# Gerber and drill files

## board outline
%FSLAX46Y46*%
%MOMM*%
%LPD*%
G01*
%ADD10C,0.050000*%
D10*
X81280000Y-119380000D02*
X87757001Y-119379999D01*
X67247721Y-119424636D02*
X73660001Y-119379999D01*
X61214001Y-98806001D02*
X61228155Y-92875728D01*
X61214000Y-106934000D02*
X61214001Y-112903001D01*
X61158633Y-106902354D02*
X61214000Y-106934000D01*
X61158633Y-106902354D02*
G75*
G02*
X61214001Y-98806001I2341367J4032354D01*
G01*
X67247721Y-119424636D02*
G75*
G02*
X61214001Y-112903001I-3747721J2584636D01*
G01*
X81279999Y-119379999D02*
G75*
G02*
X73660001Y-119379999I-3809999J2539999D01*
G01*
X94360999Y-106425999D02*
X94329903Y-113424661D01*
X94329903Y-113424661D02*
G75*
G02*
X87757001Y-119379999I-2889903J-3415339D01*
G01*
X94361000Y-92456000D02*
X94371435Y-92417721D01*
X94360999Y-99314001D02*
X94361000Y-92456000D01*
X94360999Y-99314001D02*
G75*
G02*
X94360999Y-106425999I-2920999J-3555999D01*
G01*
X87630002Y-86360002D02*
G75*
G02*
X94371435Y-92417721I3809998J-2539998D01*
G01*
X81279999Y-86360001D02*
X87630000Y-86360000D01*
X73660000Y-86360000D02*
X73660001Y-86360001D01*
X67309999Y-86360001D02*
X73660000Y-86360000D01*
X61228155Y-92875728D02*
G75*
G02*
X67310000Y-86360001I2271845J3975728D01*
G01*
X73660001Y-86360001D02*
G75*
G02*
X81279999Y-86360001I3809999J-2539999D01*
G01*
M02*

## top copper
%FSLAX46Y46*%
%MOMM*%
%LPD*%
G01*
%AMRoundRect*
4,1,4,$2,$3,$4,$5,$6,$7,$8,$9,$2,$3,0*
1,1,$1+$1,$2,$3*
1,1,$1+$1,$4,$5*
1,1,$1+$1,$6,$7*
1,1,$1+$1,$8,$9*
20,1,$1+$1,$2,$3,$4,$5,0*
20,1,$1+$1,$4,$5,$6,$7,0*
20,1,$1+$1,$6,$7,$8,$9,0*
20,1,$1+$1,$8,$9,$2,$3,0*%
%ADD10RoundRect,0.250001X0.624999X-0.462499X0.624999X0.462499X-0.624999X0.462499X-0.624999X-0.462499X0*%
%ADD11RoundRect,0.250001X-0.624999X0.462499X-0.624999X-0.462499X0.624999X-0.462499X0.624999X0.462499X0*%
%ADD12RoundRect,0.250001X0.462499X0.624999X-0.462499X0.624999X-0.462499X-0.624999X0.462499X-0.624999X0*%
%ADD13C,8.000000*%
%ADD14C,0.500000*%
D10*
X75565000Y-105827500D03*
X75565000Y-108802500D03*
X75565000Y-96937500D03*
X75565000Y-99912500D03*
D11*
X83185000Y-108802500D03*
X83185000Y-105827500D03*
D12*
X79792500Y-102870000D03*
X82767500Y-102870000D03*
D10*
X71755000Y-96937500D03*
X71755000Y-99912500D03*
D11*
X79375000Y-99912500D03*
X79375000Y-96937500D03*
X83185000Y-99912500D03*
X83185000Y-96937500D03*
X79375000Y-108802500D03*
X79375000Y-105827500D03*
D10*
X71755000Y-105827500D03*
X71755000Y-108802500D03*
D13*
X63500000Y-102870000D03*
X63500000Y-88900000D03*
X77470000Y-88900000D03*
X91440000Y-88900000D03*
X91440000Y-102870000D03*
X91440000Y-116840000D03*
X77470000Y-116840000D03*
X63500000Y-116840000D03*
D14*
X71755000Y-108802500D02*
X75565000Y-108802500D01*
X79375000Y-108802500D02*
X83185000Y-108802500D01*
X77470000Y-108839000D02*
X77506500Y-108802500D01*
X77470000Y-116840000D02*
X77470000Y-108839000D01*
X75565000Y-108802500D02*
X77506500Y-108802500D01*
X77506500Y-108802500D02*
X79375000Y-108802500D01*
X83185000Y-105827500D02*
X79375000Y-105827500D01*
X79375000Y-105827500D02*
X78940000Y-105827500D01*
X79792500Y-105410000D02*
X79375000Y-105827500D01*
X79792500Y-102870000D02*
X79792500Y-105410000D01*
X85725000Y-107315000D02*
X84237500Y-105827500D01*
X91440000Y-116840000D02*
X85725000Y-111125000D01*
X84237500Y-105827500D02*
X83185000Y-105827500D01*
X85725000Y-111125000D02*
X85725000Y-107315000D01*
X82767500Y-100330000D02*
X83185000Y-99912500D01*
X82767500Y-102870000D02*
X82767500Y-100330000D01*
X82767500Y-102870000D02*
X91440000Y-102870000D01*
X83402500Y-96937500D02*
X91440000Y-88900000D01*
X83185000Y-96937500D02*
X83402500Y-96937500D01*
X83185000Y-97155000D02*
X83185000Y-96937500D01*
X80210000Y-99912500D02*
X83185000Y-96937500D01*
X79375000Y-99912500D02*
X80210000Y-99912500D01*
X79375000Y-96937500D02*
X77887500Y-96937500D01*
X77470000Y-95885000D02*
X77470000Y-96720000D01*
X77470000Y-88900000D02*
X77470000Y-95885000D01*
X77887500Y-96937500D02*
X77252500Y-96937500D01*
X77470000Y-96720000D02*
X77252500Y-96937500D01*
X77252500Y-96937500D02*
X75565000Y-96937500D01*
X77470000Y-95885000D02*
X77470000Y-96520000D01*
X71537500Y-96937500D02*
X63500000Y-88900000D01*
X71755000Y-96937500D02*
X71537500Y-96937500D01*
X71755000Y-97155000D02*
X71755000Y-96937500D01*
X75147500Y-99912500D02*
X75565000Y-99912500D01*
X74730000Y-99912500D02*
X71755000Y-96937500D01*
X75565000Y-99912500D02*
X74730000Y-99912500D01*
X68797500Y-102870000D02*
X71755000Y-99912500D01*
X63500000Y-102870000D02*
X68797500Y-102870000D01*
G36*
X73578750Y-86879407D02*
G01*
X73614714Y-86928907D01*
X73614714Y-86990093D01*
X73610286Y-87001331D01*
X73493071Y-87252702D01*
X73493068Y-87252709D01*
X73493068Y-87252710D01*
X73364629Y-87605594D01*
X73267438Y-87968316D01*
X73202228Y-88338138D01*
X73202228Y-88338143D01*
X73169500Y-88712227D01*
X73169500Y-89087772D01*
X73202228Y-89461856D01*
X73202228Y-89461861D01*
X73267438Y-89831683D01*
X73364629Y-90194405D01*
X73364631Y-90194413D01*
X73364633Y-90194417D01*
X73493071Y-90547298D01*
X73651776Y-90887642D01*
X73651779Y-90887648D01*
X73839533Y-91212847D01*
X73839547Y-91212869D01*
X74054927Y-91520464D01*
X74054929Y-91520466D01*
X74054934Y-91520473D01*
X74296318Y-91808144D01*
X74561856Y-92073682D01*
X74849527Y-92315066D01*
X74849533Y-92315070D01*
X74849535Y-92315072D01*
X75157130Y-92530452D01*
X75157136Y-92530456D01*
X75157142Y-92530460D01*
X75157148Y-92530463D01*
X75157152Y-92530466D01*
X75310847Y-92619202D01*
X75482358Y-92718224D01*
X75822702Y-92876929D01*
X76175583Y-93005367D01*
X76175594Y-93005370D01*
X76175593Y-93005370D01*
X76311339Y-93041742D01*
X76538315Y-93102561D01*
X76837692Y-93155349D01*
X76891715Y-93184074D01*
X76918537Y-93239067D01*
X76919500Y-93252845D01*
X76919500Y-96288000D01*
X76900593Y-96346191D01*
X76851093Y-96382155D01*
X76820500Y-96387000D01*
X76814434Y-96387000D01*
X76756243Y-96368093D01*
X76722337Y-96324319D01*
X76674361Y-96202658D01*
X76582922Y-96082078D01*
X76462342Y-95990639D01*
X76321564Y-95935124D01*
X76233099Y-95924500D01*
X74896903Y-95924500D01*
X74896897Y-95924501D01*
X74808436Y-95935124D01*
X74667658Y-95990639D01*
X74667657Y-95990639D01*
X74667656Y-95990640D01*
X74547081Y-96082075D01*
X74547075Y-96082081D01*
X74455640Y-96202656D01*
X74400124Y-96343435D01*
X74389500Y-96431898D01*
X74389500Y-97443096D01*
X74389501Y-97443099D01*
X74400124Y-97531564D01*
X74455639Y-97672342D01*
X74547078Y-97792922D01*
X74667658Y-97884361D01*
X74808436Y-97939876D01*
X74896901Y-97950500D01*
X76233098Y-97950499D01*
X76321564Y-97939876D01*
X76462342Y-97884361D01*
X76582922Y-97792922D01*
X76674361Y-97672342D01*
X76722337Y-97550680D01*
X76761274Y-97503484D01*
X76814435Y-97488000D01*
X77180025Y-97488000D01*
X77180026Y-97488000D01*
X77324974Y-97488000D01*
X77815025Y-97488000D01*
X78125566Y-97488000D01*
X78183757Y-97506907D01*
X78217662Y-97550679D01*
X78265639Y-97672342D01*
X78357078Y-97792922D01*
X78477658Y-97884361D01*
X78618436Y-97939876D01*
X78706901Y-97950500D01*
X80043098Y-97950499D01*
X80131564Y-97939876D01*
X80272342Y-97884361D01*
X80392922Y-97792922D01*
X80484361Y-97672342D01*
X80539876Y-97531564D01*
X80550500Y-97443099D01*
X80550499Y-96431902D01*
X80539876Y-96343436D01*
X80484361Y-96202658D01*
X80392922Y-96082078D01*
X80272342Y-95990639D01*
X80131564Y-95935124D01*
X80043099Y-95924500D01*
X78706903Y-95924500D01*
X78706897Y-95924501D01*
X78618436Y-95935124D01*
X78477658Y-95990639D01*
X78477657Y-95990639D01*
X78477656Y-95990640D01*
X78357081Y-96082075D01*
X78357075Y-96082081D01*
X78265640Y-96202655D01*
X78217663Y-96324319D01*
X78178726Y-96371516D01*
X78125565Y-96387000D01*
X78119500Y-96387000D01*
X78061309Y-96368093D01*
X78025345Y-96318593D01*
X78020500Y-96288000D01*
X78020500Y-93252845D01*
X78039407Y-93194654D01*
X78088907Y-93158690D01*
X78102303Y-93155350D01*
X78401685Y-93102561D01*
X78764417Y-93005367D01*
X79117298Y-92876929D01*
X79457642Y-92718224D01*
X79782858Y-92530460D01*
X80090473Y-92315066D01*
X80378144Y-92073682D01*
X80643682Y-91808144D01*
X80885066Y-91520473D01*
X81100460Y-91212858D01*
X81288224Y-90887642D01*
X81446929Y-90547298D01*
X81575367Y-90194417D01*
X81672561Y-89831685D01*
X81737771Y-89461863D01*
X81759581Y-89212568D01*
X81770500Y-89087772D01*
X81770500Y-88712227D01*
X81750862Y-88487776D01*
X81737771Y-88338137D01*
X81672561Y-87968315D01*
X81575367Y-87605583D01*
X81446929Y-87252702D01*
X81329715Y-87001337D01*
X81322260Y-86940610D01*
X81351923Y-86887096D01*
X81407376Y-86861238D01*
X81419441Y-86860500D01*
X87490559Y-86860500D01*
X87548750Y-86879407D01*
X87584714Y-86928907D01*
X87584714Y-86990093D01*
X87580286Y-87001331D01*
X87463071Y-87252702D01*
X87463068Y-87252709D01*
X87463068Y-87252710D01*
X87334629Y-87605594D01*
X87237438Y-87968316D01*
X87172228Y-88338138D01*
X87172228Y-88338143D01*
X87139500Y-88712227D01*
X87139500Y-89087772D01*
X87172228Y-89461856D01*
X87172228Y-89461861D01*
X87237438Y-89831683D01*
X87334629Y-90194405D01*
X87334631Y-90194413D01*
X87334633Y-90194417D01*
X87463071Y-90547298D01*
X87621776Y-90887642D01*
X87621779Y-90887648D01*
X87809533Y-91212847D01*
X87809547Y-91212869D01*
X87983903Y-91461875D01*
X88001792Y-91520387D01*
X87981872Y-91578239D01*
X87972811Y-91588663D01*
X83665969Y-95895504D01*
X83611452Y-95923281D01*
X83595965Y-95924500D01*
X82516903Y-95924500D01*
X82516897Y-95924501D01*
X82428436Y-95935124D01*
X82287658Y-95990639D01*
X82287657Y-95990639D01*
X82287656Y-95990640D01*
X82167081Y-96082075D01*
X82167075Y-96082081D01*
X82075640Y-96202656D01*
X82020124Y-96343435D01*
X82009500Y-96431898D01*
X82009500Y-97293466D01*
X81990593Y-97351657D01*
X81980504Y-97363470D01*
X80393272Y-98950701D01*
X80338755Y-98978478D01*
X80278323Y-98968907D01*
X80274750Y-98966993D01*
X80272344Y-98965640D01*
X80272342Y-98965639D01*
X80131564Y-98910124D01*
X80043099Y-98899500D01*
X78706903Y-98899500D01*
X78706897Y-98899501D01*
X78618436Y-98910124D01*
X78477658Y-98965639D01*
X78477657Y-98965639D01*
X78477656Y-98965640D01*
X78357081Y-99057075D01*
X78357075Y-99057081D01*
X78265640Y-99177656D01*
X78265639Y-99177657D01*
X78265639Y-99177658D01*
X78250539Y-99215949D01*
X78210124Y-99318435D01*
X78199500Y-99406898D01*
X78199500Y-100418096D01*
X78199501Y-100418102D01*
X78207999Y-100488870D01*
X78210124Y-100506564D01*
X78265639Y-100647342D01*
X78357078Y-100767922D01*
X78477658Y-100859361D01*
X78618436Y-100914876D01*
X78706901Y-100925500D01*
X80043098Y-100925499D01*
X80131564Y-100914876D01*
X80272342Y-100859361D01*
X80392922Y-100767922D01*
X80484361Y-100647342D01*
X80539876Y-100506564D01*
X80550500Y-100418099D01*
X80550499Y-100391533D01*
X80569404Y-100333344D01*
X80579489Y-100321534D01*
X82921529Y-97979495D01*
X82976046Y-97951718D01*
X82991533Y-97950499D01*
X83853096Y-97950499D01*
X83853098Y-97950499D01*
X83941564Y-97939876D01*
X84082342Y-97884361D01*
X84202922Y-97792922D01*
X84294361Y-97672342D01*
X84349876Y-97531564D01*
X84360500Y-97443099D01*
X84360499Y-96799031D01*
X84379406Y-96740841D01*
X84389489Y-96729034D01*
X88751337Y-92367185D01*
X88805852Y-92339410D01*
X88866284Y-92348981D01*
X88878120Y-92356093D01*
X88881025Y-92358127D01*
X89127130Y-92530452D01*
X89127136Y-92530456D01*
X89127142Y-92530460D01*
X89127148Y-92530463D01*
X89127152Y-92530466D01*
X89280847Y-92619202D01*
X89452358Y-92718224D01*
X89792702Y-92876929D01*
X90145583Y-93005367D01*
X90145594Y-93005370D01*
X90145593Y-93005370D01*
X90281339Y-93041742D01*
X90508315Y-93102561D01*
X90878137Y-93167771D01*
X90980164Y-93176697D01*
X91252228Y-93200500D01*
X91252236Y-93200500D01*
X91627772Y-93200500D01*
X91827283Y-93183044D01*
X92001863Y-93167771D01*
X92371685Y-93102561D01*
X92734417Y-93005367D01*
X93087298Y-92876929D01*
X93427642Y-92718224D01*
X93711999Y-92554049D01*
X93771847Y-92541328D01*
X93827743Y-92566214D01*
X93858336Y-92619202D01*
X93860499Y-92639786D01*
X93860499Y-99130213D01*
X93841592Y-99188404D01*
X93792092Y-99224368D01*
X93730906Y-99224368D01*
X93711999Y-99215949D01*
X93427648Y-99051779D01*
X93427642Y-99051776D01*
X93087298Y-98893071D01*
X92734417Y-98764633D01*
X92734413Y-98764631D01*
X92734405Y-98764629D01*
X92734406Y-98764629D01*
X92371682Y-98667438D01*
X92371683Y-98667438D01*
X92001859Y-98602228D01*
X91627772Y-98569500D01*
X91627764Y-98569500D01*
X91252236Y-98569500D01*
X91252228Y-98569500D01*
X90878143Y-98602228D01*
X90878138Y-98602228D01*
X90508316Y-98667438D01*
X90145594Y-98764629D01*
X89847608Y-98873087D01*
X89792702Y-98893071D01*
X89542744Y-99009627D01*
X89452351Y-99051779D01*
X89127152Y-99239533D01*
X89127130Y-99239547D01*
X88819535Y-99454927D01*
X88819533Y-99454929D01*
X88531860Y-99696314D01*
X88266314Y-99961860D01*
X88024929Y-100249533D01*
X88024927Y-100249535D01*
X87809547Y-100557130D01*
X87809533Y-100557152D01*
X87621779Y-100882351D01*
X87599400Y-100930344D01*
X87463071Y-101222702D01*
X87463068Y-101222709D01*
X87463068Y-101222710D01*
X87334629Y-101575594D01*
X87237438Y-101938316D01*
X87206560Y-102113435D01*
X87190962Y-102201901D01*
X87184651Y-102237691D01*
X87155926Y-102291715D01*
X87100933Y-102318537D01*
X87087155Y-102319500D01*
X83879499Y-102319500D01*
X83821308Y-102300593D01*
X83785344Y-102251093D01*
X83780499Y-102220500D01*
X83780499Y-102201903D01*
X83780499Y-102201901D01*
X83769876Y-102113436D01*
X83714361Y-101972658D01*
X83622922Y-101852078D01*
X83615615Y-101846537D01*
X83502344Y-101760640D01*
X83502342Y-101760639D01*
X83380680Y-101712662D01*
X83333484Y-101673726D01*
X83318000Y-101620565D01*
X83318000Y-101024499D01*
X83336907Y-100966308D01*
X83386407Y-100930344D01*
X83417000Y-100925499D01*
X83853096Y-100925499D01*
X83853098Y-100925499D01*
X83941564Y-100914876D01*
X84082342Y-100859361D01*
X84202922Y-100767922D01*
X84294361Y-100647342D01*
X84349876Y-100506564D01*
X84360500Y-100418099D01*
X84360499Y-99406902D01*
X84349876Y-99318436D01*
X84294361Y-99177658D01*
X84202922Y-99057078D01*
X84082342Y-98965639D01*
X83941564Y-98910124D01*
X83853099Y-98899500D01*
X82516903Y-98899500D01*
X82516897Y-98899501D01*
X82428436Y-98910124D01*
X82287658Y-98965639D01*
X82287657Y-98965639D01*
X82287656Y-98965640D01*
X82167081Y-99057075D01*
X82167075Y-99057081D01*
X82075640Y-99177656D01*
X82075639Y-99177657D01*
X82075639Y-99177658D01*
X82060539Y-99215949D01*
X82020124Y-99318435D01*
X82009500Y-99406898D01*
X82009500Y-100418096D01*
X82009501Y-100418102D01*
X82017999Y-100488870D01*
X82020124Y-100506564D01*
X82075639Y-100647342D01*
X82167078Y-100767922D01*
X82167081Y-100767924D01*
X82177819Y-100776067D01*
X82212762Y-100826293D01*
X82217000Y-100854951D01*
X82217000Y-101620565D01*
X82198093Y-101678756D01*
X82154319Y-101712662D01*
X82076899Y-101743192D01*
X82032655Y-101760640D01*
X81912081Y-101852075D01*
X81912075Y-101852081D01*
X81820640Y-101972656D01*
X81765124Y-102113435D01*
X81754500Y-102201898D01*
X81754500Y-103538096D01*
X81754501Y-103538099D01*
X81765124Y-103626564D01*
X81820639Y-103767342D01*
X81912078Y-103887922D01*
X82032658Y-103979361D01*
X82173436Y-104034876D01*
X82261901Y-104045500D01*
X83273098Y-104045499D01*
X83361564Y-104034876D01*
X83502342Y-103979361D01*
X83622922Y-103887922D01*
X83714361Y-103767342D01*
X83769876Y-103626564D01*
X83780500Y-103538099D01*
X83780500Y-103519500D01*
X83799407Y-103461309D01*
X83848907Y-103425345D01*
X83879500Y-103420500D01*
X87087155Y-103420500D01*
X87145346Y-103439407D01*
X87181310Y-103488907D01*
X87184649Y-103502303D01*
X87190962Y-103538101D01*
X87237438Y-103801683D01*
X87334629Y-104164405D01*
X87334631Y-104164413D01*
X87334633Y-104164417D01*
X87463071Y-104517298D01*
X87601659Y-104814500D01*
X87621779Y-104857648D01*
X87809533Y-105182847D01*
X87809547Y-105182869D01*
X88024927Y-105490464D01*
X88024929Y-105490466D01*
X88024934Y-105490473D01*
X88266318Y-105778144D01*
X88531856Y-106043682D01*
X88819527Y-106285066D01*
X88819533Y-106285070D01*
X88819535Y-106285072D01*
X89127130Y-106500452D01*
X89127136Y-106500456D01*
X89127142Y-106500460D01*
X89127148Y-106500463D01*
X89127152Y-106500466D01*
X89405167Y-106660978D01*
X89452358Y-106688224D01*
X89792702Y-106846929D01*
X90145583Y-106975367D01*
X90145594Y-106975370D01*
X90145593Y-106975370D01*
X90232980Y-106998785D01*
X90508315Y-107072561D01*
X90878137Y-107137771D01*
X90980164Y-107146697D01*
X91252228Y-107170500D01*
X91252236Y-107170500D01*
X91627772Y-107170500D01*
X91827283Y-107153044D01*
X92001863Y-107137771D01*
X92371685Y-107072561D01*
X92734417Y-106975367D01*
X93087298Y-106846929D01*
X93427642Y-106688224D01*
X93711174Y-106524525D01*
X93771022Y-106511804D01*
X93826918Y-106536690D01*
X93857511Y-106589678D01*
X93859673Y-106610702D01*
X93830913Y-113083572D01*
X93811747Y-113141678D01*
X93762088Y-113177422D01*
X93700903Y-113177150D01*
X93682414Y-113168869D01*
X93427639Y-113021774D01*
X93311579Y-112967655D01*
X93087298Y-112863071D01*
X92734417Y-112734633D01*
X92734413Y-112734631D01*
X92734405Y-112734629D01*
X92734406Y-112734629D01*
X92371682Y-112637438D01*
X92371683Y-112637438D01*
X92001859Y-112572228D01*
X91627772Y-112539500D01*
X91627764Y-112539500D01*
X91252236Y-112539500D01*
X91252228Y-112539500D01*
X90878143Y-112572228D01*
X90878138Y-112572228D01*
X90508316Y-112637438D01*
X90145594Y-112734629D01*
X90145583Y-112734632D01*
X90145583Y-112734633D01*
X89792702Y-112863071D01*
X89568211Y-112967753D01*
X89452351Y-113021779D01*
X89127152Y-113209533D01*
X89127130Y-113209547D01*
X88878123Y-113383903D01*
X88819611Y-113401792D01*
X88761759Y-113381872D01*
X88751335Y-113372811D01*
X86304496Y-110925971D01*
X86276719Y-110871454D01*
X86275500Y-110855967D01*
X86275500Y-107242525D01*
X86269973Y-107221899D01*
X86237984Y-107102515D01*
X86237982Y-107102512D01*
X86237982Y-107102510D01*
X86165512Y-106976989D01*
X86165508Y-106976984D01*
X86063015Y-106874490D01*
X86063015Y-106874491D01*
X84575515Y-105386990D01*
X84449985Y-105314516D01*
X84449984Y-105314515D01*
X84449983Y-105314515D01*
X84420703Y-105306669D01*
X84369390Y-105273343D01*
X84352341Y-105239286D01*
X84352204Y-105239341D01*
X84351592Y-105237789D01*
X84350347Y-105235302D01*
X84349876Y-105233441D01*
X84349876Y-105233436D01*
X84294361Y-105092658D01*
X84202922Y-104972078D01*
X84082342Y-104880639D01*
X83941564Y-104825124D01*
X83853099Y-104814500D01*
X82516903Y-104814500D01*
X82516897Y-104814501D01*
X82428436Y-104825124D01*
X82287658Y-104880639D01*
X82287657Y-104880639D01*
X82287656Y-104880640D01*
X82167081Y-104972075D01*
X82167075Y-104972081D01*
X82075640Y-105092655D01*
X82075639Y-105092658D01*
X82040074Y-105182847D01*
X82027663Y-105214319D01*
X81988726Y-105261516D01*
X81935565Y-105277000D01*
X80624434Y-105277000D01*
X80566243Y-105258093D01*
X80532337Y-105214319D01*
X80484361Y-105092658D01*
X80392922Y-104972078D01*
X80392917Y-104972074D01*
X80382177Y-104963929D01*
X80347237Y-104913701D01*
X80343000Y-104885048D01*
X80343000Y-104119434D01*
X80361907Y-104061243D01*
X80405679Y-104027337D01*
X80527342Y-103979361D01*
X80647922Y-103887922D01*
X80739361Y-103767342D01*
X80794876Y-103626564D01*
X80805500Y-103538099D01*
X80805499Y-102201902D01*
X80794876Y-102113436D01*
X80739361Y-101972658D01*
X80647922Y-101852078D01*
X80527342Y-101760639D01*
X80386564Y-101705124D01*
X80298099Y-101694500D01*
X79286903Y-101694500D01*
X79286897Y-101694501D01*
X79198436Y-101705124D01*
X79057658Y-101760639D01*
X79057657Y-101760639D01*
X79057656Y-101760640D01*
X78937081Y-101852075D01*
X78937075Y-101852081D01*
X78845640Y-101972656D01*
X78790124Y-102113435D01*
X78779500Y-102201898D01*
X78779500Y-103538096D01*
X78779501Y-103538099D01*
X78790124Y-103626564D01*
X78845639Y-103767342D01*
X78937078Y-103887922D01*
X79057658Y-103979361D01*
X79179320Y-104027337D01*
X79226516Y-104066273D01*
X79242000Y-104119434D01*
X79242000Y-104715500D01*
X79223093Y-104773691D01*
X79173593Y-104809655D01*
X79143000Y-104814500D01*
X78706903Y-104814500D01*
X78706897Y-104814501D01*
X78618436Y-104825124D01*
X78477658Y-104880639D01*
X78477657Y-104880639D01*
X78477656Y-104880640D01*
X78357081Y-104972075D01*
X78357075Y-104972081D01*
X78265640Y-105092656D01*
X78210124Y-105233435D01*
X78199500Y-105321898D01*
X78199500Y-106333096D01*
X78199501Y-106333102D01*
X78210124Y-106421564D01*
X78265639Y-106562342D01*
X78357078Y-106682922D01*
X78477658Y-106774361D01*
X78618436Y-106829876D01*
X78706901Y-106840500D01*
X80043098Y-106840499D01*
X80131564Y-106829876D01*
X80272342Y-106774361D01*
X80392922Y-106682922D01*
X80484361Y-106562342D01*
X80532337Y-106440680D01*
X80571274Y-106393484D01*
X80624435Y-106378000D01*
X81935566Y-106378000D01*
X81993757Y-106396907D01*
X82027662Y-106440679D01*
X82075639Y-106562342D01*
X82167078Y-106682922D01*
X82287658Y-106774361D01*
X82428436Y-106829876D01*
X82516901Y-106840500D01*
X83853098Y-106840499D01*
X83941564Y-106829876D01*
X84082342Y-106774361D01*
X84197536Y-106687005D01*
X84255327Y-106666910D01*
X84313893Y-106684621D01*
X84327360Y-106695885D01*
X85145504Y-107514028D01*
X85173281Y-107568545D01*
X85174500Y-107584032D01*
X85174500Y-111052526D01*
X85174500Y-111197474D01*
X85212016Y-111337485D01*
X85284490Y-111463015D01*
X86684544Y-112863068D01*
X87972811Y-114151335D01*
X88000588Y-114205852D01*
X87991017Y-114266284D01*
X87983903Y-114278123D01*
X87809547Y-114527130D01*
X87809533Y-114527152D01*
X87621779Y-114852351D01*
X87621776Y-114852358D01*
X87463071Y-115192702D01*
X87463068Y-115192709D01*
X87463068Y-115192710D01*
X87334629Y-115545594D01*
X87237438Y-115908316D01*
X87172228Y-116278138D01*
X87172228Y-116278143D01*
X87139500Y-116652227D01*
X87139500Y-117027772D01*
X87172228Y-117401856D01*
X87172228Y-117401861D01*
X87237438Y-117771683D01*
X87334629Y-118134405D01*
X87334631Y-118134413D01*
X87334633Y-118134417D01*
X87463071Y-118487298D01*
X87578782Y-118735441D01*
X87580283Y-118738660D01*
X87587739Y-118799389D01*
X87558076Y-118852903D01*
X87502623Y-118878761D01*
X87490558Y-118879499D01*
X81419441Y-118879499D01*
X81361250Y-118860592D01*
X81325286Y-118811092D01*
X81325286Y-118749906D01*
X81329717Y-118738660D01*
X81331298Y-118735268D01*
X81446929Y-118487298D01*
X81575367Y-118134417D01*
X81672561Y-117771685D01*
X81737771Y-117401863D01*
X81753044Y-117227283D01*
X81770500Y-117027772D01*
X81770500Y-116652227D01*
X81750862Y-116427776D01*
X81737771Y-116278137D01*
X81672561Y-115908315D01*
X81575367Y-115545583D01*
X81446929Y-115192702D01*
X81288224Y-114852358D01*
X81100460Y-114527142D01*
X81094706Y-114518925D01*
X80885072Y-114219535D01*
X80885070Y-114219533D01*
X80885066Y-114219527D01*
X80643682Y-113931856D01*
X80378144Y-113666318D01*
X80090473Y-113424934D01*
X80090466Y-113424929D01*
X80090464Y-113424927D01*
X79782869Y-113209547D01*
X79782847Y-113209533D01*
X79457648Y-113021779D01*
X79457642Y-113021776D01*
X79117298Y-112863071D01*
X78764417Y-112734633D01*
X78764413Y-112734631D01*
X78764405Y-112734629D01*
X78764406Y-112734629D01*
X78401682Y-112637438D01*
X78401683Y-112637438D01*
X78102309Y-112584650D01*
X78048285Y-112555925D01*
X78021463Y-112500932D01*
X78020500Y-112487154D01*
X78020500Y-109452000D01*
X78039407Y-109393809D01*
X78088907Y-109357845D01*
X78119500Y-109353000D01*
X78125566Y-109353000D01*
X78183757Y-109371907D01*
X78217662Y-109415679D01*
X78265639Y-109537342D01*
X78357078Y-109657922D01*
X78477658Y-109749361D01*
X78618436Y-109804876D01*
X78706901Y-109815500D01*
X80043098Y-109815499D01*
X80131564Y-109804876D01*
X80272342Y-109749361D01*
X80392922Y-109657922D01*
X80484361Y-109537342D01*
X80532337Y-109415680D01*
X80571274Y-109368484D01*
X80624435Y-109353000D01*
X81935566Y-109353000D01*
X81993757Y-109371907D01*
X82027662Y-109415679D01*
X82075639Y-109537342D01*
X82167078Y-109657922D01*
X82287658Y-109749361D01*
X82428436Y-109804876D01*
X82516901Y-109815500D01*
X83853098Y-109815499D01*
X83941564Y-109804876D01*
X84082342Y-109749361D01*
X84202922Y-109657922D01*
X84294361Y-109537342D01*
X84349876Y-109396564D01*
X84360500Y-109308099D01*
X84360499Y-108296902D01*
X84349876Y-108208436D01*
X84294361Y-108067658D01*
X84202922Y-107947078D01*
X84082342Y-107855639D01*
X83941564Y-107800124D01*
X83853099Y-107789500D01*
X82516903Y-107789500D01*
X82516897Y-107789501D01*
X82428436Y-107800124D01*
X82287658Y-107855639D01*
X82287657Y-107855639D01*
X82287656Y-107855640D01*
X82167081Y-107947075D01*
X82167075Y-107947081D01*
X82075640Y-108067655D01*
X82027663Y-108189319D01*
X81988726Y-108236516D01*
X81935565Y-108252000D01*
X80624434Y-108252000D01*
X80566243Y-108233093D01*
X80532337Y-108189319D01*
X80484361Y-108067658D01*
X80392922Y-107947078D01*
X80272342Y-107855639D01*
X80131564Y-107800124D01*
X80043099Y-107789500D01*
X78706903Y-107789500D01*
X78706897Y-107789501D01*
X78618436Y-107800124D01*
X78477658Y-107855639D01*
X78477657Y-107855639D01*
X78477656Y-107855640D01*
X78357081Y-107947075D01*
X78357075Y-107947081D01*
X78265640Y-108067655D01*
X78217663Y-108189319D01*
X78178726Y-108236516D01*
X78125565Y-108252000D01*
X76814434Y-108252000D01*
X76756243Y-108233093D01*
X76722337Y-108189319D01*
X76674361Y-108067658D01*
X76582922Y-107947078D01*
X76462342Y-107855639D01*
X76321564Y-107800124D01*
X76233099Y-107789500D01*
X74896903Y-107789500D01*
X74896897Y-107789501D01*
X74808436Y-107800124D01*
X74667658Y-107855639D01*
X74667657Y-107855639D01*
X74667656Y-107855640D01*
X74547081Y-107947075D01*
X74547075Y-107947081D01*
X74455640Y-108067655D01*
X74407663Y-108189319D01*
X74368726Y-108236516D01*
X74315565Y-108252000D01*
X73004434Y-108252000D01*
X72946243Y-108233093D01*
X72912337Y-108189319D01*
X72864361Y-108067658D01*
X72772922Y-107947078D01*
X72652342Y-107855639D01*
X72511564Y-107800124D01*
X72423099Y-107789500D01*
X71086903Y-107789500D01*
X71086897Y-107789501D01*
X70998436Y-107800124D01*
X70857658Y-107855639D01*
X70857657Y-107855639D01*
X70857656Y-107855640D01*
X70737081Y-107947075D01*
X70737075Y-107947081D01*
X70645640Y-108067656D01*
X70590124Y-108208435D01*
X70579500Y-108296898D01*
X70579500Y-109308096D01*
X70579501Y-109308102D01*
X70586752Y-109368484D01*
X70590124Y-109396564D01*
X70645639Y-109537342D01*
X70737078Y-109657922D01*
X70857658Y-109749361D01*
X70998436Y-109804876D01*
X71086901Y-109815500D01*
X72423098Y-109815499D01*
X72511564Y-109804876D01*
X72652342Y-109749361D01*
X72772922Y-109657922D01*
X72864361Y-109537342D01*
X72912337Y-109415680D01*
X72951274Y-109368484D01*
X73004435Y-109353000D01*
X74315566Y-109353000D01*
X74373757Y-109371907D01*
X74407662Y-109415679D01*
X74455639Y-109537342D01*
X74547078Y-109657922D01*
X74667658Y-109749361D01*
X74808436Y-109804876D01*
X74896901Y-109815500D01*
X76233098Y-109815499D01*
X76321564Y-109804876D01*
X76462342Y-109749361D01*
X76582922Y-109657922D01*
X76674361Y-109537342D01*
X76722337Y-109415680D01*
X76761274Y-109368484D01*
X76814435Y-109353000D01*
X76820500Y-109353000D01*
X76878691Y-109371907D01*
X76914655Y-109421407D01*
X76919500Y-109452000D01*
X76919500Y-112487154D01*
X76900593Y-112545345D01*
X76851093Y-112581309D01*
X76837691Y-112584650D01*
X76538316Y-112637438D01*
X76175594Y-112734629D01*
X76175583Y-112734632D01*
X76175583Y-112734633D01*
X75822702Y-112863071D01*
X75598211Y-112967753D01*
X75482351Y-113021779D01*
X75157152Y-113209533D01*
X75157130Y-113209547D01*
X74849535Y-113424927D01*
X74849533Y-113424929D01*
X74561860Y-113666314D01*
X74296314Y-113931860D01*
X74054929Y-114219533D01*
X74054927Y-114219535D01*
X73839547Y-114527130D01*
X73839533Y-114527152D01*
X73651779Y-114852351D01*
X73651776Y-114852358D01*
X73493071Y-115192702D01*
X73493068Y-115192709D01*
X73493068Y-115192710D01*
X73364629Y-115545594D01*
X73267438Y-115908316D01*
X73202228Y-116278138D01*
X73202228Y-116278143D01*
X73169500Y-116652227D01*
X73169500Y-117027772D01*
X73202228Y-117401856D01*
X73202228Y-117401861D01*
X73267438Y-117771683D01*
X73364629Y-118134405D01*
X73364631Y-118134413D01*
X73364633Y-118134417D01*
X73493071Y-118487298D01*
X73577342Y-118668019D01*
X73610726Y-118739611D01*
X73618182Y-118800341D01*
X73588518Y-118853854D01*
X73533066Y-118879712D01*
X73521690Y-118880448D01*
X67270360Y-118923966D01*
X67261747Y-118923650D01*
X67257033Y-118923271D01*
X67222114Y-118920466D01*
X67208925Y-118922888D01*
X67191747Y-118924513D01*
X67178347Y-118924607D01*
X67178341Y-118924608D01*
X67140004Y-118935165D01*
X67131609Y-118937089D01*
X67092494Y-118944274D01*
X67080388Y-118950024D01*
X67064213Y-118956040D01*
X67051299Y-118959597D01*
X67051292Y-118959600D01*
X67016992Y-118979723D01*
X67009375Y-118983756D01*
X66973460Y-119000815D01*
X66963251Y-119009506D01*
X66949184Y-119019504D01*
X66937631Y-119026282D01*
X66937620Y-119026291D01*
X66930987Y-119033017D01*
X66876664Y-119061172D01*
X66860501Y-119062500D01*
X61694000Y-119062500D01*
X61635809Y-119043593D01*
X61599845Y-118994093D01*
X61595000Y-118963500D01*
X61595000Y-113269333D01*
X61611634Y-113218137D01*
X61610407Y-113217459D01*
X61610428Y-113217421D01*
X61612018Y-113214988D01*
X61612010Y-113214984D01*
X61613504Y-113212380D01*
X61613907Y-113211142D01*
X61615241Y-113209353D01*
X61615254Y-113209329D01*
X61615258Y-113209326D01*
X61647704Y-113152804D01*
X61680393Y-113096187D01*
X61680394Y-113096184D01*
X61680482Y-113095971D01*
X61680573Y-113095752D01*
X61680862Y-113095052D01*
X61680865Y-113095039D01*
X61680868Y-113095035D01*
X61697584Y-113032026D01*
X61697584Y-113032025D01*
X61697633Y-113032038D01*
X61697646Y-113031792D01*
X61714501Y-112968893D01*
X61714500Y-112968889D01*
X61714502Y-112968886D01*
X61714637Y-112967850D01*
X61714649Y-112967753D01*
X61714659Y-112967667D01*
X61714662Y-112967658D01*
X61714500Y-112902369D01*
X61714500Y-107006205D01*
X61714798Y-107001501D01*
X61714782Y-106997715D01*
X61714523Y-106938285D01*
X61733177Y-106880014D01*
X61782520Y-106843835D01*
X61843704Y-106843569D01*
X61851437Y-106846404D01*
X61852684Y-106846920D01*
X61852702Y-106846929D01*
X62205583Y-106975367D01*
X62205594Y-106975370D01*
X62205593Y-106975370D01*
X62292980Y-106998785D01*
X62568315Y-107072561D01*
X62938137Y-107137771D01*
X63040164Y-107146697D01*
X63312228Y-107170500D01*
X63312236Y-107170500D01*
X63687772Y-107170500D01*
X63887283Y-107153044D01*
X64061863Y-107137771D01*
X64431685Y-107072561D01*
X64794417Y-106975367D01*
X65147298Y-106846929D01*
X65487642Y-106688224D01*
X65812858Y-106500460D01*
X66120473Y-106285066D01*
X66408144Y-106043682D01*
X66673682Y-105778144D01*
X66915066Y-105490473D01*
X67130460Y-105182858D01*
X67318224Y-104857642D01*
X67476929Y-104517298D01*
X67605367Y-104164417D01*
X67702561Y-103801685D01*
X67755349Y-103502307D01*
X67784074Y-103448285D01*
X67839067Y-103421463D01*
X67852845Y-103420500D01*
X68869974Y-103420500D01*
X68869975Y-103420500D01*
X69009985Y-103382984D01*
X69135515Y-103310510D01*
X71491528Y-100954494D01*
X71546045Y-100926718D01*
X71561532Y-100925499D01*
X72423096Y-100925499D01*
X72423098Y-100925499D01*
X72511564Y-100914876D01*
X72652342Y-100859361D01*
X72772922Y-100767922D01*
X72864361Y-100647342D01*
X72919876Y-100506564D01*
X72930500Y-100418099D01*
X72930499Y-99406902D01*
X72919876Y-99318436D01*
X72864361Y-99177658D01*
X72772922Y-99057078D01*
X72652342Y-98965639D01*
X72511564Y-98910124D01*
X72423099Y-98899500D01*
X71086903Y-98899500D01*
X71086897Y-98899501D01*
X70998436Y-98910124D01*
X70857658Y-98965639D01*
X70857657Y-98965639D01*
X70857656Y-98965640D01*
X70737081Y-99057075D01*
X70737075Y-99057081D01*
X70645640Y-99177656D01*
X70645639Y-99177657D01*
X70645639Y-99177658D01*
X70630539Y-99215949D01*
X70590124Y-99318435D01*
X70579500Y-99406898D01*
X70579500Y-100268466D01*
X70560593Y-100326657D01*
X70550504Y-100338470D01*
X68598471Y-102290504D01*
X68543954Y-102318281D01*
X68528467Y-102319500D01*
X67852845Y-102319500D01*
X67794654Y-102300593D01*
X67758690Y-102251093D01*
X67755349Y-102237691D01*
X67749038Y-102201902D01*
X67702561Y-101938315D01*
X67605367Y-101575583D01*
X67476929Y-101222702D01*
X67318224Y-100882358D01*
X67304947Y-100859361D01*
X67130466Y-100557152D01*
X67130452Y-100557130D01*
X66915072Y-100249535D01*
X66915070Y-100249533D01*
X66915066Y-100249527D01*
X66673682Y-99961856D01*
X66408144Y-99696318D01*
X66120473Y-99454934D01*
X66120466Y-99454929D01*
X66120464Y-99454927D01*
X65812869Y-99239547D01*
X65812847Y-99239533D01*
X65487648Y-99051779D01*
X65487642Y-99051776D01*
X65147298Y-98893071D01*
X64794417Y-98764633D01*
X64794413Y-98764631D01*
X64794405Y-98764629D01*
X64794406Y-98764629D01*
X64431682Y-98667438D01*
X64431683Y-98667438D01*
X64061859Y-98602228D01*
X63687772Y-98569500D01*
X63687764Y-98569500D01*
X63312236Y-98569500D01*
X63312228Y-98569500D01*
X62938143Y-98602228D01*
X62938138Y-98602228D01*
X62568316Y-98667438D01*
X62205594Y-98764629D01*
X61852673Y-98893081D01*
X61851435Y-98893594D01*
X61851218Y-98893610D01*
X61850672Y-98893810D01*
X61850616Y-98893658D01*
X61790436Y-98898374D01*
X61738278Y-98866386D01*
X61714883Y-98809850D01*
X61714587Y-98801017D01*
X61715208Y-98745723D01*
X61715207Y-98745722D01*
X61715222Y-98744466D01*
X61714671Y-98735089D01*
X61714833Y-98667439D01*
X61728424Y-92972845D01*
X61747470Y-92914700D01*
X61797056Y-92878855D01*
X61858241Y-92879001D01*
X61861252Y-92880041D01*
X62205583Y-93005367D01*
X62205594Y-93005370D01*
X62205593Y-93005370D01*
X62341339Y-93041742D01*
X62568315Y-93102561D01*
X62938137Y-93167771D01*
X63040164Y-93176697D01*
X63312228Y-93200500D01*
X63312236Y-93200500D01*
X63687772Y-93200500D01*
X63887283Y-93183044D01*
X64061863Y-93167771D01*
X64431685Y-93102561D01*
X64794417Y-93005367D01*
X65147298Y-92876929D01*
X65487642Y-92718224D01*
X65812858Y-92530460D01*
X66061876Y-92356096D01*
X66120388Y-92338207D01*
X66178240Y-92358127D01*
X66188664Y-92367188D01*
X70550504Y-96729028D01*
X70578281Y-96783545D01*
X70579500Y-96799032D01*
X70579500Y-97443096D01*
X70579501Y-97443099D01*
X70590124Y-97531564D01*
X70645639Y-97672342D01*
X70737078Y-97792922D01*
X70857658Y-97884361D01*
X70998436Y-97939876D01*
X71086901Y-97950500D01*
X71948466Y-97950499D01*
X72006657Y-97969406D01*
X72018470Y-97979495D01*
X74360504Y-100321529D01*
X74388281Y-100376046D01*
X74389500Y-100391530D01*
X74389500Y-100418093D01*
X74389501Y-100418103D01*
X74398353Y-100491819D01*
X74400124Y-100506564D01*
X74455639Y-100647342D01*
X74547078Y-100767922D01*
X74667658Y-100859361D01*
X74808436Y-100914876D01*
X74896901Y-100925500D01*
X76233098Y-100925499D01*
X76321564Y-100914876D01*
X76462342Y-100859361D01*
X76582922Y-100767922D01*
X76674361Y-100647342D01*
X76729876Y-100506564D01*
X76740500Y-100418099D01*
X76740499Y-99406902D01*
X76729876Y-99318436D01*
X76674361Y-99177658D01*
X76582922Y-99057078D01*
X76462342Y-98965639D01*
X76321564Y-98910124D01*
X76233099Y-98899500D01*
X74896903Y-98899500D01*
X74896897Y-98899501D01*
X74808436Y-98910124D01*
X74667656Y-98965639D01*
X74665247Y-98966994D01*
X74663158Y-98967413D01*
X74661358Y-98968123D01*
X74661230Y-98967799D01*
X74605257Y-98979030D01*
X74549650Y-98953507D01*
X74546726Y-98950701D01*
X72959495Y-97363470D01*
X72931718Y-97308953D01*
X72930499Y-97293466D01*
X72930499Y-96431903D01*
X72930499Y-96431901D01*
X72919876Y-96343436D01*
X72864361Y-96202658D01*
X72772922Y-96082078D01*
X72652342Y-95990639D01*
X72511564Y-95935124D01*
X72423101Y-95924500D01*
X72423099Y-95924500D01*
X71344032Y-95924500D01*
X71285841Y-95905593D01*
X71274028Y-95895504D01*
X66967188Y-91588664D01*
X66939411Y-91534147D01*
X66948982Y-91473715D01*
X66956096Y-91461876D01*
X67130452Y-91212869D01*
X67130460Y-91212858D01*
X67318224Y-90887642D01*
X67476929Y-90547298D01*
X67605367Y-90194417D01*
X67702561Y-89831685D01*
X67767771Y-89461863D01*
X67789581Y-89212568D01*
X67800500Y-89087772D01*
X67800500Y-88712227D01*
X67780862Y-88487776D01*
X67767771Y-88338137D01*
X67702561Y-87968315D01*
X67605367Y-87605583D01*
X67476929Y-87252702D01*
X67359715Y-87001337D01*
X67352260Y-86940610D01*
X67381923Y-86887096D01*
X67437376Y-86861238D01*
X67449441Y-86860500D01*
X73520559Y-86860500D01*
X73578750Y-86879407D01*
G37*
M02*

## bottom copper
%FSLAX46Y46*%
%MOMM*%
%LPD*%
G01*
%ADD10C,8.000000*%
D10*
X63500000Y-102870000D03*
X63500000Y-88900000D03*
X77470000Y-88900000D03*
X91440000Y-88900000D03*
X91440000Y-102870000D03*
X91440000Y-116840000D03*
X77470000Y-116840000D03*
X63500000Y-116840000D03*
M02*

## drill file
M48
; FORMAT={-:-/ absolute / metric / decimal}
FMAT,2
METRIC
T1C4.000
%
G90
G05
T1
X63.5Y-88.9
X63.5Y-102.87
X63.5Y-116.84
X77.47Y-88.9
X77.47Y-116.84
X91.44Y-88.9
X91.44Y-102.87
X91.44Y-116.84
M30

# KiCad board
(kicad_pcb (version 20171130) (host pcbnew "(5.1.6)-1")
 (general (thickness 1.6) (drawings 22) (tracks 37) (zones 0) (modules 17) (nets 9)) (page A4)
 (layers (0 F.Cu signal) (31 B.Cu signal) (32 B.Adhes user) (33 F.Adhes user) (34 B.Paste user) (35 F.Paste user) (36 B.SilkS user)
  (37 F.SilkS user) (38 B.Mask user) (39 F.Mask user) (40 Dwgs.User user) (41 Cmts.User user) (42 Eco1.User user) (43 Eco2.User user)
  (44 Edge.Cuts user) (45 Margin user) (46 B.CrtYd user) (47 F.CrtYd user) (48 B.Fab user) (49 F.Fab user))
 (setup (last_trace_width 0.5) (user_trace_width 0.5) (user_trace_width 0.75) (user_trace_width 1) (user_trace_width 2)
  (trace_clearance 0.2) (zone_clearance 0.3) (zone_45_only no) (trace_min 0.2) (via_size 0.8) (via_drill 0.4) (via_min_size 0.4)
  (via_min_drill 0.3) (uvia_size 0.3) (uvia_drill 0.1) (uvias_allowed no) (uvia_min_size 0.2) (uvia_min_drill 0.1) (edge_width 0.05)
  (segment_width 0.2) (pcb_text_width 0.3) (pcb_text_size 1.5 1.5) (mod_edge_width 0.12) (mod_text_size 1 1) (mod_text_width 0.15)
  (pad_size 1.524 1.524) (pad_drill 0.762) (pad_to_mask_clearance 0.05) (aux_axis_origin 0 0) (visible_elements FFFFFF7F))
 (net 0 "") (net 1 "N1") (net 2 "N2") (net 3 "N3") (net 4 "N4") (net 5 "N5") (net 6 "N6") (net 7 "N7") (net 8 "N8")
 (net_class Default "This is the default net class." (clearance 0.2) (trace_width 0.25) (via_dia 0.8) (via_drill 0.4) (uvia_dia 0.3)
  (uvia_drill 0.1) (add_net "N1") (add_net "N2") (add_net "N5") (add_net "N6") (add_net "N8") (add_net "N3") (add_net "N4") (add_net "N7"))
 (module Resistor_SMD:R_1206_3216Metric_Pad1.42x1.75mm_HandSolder (layer F.Cu) (at 75.565 107.315 90)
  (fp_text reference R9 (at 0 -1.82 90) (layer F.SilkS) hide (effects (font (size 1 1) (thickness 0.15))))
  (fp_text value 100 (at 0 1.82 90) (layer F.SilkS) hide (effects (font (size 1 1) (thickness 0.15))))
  (pad 2 smd roundrect (at 1.4875 0 90) (size 1.425 1.75) (layers F.Cu F.Paste F.Mask) (roundrect_rratio 0.175439) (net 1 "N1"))
  (pad 1 smd roundrect (at -1.4875 0 90) (size 1.425 1.75) (layers F.Cu F.Paste F.Mask) (roundrect_rratio 0.175439) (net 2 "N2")))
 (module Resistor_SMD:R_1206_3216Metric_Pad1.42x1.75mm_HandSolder (layer F.Cu) (at 75.565 98.425 90)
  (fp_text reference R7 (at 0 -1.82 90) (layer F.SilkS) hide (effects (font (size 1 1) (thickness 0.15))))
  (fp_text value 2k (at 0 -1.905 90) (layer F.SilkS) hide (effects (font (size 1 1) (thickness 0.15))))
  (pad 2 smd roundrect (at 1.4875 0 90) (size 1.425 1.75) (layers F.Cu F.Paste F.Mask) (roundrect_rratio 0.175439) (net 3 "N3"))
  (pad 1 smd roundrect (at -1.4875 0 90) (size 1.425 1.75) (layers F.Cu F.Paste F.Mask) (roundrect_rratio 0.175439) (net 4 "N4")))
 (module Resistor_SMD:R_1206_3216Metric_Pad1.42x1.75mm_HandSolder (layer F.Cu) (at 83.185 107.315 270)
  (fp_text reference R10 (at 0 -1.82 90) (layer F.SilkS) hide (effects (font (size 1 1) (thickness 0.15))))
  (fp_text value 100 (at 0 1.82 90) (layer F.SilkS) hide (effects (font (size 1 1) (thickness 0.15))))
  (pad 2 smd roundrect (at 1.4875 0 270) (size 1.425 1.75) (layers F.Cu F.Paste F.Mask) (roundrect_rratio 0.175439) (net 2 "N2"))
  (pad 1 smd roundrect (at -1.4875 0 270) (size 1.425 1.75) (layers F.Cu F.Paste F.Mask) (roundrect_rratio 0.175439) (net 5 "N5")))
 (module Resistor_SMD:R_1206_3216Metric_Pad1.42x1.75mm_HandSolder (layer F.Cu) (at 81.28 102.87 180)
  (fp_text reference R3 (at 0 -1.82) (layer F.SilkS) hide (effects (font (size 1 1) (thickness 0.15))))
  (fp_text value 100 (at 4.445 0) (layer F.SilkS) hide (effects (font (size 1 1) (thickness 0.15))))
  (pad 2 smd roundrect (at 1.4875 0 180) (size 1.425 1.75) (layers F.Cu F.Paste F.Mask) (roundrect_rratio 0.175439) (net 5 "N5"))
  (pad 1 smd roundrect (at -1.4875 0 180) (size 1.425 1.75) (layers F.Cu F.Paste F.Mask) (roundrect_rratio 0.175439) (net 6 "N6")))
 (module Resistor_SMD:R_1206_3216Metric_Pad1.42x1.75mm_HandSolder (layer F.Cu) (at 71.755 98.425 90)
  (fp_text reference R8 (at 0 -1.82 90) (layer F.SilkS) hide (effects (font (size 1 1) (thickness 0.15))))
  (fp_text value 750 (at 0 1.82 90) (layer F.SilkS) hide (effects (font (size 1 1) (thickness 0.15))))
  (pad 2 smd roundrect (at 1.4875 0 90) (size 1.425 1.75) (layers F.Cu F.Paste F.Mask) (roundrect_rratio 0.175439) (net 4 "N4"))
  (pad 1 smd roundrect (at -1.4875 0 90) (size 1.425 1.75) (layers F.Cu F.Paste F.Mask) (roundrect_rratio 0.175439) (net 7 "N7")))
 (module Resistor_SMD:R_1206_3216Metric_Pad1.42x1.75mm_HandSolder (layer F.Cu) (at 79.375 98.425 270)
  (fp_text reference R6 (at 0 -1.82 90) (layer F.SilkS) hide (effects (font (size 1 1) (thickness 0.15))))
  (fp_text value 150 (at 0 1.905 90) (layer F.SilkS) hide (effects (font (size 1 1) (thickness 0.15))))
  (pad 2 smd roundrect (at 1.4875 0 270) (size 1.425 1.75) (layers F.Cu F.Paste F.Mask) (roundrect_rratio 0.175439) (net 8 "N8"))
  (pad 1 smd roundrect (at -1.4875 0 270) (size 1.425 1.75) (layers F.Cu F.Paste F.Mask) (roundrect_rratio 0.175439) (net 3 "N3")))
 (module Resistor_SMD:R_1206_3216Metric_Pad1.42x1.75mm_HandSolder (layer F.Cu) (at 83.185 98.425 270)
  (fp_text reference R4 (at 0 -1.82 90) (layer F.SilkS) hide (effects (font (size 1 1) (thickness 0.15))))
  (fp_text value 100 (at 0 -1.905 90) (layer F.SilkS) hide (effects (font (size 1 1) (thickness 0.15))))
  (pad 2 smd roundrect (at 1.4875 0 270) (size 1.425 1.75) (layers F.Cu F.Paste F.Mask) (roundrect_rratio 0.175439) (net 6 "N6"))
  (pad 1 smd roundrect (at -1.4875 0 270) (size 1.425 1.75) (layers F.Cu F.Paste F.Mask) (roundrect_rratio 0.175439) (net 8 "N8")))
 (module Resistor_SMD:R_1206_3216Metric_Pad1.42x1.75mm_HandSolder (layer F.Cu) (at 79.375 107.315 270)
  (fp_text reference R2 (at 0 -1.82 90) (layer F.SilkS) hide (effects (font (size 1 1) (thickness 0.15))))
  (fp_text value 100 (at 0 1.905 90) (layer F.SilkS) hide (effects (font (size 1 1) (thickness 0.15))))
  (pad 2 smd roundrect (at 1.4875 0 270) (size 1.425 1.75) (layers F.Cu F.Paste F.Mask) (roundrect_rratio 0.175439) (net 2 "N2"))
  (pad 1 smd roundrect (at -1.4875 0 270) (size 1.425 1.75) (layers F.Cu F.Paste F.Mask) (roundrect_rratio 0.175439) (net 5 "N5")))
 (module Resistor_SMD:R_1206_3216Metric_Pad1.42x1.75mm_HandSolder (layer F.Cu) (at 71.755 107.315 90)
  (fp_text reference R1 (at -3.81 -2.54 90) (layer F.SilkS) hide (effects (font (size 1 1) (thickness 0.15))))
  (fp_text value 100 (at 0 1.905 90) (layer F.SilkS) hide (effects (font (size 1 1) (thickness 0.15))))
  (pad 2 smd roundrect (at 1.4875 0 90) (size 1.425 1.75) (layers F.Cu F.Paste F.Mask) (roundrect_rratio 0.175439) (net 1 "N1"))
  (pad 1 smd roundrect (at -1.4875 0 90) (size 1.425 1.75) (layers F.Cu F.Paste F.Mask) (roundrect_rratio 0.175439) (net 2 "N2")))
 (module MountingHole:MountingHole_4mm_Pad (layer F.Cu) (at 63.5 102.87)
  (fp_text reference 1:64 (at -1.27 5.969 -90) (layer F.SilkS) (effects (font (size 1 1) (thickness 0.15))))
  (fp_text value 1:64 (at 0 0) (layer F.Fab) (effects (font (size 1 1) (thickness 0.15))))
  (pad 1 thru_hole circle (at 0 0) (size 8 8) (drill 4) (layers *.Cu *.Mask) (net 7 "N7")))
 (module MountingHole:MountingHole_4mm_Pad (layer F.Cu) (at 63.5 88.9)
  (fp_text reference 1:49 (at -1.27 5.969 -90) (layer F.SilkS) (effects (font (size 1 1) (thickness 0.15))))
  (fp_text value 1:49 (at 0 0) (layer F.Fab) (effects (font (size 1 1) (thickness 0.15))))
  (pad 1 thru_hole circle (at 0 0) (size 8 8) (drill 4) (layers *.Cu *.Mask) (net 4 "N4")))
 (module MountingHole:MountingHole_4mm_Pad (layer F.Cu) (at 77.47 88.9)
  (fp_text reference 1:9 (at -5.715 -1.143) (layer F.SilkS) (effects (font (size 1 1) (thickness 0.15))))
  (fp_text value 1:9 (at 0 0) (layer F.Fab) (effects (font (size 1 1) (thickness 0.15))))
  (pad 1 thru_hole circle (at 0 0) (size 8 8) (drill 4) (layers *.Cu *.Mask) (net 3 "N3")))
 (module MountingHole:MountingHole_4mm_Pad (layer F.Cu) (at 91.44 88.9)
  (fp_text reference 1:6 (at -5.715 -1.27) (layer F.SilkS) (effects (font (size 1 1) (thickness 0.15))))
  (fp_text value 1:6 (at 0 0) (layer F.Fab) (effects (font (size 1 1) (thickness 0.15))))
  (pad 1 thru_hole circle (at 0 0) (size 8 8) (drill 4) (layers *.Cu *.Mask) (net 8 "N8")))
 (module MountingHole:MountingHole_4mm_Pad (layer F.Cu) (at 91.44 102.87)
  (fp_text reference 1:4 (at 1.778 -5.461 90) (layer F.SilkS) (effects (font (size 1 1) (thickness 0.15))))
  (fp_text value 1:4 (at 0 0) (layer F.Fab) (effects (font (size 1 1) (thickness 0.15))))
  (pad 1 thru_hole circle (at 0 0) (size 8 8) (drill 4) (layers *.Cu *.Mask) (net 6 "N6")))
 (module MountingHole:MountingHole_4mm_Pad (layer F.Cu) (at 91.44 116.84)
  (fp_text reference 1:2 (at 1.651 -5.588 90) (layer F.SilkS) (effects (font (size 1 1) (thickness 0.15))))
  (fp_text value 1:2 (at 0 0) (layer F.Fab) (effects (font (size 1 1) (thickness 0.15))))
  (pad 1 thru_hole circle (at 0 0) (size 8 8) (drill 4) (layers *.Cu *.Mask) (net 5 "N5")))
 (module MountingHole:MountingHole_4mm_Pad (layer F.Cu) (at 77.47 116.84)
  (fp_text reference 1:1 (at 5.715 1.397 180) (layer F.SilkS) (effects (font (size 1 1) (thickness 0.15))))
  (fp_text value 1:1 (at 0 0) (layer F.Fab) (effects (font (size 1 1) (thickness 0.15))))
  (pad 1 thru_hole circle (at 0 0) (size 8 8) (drill 4) (layers *.Cu *.Mask) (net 2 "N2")))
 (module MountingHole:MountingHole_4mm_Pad (layer F.Cu) (at 63.5 116.84)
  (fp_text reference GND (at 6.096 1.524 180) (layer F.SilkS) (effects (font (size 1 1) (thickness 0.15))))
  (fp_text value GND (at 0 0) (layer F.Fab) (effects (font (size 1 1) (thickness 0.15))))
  (pad 1 thru_hole circle (at 0 0) (size 8 8) (drill 4) (layers *.Cu *.Mask) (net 1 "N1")))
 (gr_line (start 81.28 119.38) (end 87.757001 119.379999) (layer Edge.Cuts) (width 0.05))
 (gr_line (start 67.247721 119.424636) (end 73.660001 119.379999) (layer Edge.Cuts) (width 0.05))
 (gr_line (start 61.214001 98.806001) (end 61.228155 92.875728) (layer Edge.Cuts) (width 0.05))
 (gr_line (start 61.214 106.934) (end 61.214001 112.903001) (layer Edge.Cuts) (width 0.05))
 (gr_line (start 61.158633 106.902354) (end 61.214 106.934) (layer Edge.Cuts) (width 0.05))
 (gr_arc (start 63.5 102.87) (end 61.214001 98.806001) (angle -120.5008609) (layer Edge.Cuts) (width 0.05))
 (gr_arc (start 63.5 116.84) (end 61.214001 112.903001) (angle -205.2663258) (layer Edge.Cuts) (width 0.05))
 (gr_arc (start 77.47 116.84) (end 73.660001 119.379999) (angle -112.6198649) (layer Edge.Cuts) (width 0.05))
 (gr_line (start 94.360999 106.425999) (end 94.329903 113.424661) (layer Edge.Cuts) (width 0.05))
 (gr_arc (start 91.44 116.84) (end 87.757001 119.379999) (angle -195.171353) (layer Edge.Cuts) (width 0.05))
 (gr_line (start 94.361 92.456) (end 94.371435 92.417721) (layer Edge.Cuts) (width 0.05))
 (gr_line (start 94.360999 99.314001) (end 94.361 92.456) (layer Edge.Cuts) (width 0.05))
 (gr_arc (start 91.44 102.87) (end 94.360999 106.425999) (angle -101.1986787) (layer Edge.Cuts) (width 0.05))
 (gr_arc (start 91.44 88.9) (end 94.371435 92.417721) (angle -196.5043552) (layer Edge.Cuts) (width 0.05))
 (gr_line (start 81.279999 86.360001) (end 87.63 86.36) (layer Edge.Cuts) (width 0.05))
 (gr_line (start 73.66 86.36) (end 73.660001 86.360001) (layer Edge.Cuts) (width 0.05))
 (gr_line (start 67.309999 86.360001) (end 73.66 86.36) (layer Edge.Cuts) (width 0.05))
 (gr_arc (start 63.5 88.9) (end 67.309999 86.360001) (angle -206.5650512) (layer Edge.Cuts) (width 0.05))
 (gr_arc (start 77.47 88.9) (end 81.279999 86.360001) (angle -112.6198649) (layer Edge.Cuts) (width 0.05))
 (segment (start 71.755 108.8025) (end 75.565 108.8025) (width 0.5) (layer F.Cu) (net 2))
 (segment (start 79.375 108.8025) (end 83.185 108.8025) (width 0.5) (layer F.Cu) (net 2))
 (segment (start 77.47 108.839) (end 77.5065 108.8025) (width 0.5) (layer F.Cu) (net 2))
 (segment (start 77.47 116.84) (end 77.47 108.839) (width 0.5) (layer F.Cu) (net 2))
 (segment (start 75.565 108.8025) (end 77.5065 108.8025) (width 0.5) (layer F.Cu) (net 2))
 (segment (start 77.5065 108.8025) (end 79.375 108.8025) (width 0.5) (layer F.Cu) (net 2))
 (segment (start 83.185 105.8275) (end 79.375 105.8275) (width 0.5) (layer F.Cu) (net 5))
 (segment (start 79.375 105.8275) (end 78.94 105.8275) (width 0.5) (layer F.Cu) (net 5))
 (segment (start 79.7925 105.41) (end 79.375 105.8275) (width 0.5) (layer F.Cu) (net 5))
 (segment (start 79.7925 102.87) (end 79.7925 105.41) (width 0.5) (layer F.Cu) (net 5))
 (segment (start 85.725 107.315) (end 84.2375 105.8275) (width 0.5) (layer F.Cu) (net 5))
 (segment (start 91.44 116.84) (end 85.725 111.125) (width 0.5) (layer F.Cu) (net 5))
 (segment (start 84.2375 105.8275) (end 83.185 105.8275) (width 0.5) (layer F.Cu) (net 5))
 (segment (start 85.725 111.125) (end 85.725 107.315) (width 0.5) (layer F.Cu) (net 5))
 (segment (start 82.7675 100.33) (end 83.185 99.9125) (width 0.5) (layer F.Cu) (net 6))
 (segment (start 82.7675 102.87) (end 82.7675 100.33) (width 0.5) (layer F.Cu) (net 6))
 (segment (start 82.7675 102.87) (end 91.44 102.87) (width 0.5) (layer F.Cu) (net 6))
 (segment (start 83.4025 96.9375) (end 91.44 88.9) (width 0.5) (layer F.Cu) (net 8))
 (segment (start 83.185 96.9375) (end 83.4025 96.9375) (width 0.5) (layer F.Cu) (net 8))
 (segment (start 83.185 97.155) (end 83.185 96.9375) (width 0.5) (layer F.Cu) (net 8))
 (segment (start 80.21 99.9125) (end 83.185 96.9375) (width 0.5) (layer F.Cu) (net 8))
 (segment (start 79.375 99.9125) (end 80.21 99.9125) (width 0.5) (layer F.Cu) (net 8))
 (segment (start 79.375 96.9375) (end 77.8875 96.9375) (width 0.5) (layer F.Cu) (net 3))
 (segment (start 77.47 95.885) (end 77.47 96.72) (width 0.5) (layer F.Cu) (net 3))
 (segment (start 77.47 88.9) (end 77.47 95.885) (width 0.5) (layer F.Cu) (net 3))
 (segment (start 77.8875 96.9375) (end 77.2525 96.9375) (width 0.5) (layer F.Cu) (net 3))
 (segment (start 77.47 96.72) (end 77.2525 96.9375) (width 0.5) (layer F.Cu) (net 3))
 (segment (start 77.2525 96.9375) (end 75.565 96.9375) (width 0.5) (layer F.Cu) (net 3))
 (segment (start 77.47 95.885) (end 77.47 96.52) (width 0.5) (layer F.Cu) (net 3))
 (segment (start 71.5375 96.9375) (end 63.5 88.9) (width 0.5) (layer F.Cu) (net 4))
 (segment (start 71.755 96.9375) (end 71.5375 96.9375) (width 0.5) (layer F.Cu) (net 4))
 (segment (start 71.755 97.155) (end 71.755 96.9375) (width 0.5) (layer F.Cu) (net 4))
 (segment (start 75.1475 99.9125) (end 75.565 99.9125) (width 0.5) (layer F.Cu) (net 4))
 (segment (start 74.73 99.9125) (end 71.755 96.9375) (width 0.5) (layer F.Cu) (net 4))
 (segment (start 75.565 99.9125) (end 74.73 99.9125) (width 0.5) (layer F.Cu) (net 4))
 (segment (start 68.7975 102.87) (end 71.755 99.9125) (width 0.5) (layer F.Cu) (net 7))
 (segment (start 63.5 102.87) (end 68.7975 102.87) (width 0.5) (layer F.Cu) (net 7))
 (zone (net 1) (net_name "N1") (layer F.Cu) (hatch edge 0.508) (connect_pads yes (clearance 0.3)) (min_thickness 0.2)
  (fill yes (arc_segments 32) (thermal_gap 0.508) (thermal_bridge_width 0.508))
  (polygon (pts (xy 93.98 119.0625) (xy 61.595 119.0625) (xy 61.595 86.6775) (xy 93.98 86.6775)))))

